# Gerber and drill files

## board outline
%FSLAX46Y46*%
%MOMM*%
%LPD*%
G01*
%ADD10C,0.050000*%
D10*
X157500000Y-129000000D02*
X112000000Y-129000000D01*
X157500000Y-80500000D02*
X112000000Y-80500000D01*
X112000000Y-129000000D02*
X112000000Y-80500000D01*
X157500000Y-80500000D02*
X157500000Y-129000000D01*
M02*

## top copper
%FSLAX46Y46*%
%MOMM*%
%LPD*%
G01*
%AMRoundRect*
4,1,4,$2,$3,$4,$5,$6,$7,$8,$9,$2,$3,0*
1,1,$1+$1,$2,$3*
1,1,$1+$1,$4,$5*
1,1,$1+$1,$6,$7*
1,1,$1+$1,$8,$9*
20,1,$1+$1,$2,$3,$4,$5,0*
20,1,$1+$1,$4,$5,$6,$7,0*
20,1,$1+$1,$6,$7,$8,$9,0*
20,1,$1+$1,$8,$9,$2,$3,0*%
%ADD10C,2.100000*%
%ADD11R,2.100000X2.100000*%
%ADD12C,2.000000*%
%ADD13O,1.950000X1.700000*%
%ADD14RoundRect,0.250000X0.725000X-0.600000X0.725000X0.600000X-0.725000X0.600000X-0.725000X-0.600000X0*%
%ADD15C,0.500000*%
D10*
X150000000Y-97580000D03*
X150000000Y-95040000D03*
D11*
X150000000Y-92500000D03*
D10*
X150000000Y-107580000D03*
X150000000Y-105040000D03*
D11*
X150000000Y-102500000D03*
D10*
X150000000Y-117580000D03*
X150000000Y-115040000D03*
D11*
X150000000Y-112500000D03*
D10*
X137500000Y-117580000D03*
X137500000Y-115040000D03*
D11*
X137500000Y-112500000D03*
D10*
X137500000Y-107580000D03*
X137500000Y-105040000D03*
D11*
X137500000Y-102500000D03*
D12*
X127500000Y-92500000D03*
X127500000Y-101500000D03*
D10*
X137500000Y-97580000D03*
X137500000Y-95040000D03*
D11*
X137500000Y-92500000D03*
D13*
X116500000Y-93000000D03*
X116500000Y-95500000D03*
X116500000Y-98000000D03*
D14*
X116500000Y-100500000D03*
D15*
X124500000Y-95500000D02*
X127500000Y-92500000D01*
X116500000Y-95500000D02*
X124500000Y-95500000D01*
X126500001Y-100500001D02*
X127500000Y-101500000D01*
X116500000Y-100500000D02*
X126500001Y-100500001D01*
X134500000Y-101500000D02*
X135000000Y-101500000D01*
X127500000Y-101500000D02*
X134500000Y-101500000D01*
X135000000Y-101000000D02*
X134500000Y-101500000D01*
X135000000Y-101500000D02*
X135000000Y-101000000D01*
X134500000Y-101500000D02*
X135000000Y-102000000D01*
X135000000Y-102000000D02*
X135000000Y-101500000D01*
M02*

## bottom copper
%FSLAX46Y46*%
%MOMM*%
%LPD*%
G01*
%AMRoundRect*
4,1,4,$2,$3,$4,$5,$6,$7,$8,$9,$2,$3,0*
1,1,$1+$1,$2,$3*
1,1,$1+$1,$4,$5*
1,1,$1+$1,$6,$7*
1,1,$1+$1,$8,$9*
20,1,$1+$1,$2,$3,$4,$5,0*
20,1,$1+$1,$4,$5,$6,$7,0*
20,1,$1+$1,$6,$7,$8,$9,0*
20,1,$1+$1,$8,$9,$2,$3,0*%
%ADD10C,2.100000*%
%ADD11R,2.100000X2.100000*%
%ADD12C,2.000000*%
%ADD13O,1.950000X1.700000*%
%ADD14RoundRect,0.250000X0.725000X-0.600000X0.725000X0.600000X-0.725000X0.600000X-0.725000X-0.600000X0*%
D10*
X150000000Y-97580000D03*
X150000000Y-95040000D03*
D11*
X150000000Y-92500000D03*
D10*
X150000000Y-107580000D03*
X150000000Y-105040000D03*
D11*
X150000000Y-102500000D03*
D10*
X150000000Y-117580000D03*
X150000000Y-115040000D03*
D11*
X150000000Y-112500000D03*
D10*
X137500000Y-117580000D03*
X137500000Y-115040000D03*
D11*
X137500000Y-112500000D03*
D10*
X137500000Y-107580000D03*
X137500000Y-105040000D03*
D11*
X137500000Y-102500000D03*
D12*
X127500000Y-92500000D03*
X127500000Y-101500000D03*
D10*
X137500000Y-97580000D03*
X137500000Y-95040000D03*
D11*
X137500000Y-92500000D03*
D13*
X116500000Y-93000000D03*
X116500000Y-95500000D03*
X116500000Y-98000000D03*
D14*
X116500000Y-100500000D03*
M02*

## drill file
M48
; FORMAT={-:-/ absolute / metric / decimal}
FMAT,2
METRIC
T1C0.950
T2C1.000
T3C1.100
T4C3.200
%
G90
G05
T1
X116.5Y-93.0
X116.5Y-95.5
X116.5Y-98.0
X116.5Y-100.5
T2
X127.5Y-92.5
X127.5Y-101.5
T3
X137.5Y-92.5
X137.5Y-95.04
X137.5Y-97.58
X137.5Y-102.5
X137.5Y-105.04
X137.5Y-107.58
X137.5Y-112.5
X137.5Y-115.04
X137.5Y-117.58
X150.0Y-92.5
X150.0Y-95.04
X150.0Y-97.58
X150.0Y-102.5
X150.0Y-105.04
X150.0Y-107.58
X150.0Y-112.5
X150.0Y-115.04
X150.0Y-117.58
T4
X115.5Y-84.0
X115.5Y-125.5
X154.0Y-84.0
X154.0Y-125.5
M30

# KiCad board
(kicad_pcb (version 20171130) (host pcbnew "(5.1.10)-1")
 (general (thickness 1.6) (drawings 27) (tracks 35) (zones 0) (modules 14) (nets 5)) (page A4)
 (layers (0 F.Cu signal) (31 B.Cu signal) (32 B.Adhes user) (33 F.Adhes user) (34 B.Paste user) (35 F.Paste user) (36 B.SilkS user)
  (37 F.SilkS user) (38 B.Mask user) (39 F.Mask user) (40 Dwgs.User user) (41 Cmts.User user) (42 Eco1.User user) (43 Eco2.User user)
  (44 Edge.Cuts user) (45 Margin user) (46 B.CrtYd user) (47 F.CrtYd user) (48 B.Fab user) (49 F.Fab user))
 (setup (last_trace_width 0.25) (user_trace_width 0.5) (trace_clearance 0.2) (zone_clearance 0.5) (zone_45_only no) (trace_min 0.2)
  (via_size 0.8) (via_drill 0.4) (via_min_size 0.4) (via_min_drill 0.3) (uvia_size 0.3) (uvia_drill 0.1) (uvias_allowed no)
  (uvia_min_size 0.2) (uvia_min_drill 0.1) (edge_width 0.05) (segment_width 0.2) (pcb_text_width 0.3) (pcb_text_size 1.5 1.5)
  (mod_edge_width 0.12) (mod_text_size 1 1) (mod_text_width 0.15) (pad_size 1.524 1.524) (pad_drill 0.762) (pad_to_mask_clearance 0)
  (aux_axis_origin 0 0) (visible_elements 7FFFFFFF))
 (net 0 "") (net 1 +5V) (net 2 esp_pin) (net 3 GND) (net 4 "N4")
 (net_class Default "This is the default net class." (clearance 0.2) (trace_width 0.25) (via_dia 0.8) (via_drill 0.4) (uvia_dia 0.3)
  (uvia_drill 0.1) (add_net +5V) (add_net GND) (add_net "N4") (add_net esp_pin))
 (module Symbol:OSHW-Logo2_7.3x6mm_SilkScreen (layer F.Cu) (at 137.5 124.5)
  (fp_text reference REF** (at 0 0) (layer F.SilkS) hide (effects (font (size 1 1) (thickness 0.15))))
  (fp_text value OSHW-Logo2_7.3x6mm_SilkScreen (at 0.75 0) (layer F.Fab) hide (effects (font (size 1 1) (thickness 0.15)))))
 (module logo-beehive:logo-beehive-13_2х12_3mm (layer F.Cu) (at 123 109.22)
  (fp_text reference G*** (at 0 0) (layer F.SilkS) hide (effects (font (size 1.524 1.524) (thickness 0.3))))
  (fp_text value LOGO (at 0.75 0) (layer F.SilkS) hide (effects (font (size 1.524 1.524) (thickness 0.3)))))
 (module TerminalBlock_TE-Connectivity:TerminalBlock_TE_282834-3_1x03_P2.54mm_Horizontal (layer F.Cu) (at 150 92.5 270)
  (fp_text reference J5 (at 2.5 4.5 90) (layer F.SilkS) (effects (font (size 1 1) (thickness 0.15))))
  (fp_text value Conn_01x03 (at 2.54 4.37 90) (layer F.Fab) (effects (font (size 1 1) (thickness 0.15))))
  (pad 3 thru_hole circle (at 5.08 0 270) (size 2.1 2.1) (drill 1.1) (layers *.Cu *.Mask))
  (pad 2 thru_hole circle (at 2.54 0 270) (size 2.1 2.1) (drill 1.1) (layers *.Cu *.Mask))
  (pad 1 thru_hole rect (at 0 0 270) (size 2.1 2.1) (drill 1.1) (layers *.Cu *.Mask)))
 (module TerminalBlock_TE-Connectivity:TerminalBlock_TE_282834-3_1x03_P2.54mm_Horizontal (layer F.Cu) (at 150 102.5 270)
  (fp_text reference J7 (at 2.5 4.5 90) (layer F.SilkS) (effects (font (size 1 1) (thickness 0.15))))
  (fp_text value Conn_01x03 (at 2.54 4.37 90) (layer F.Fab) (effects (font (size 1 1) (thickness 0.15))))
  (pad 3 thru_hole circle (at 5.08 0 270) (size 2.1 2.1) (drill 1.1) (layers *.Cu *.Mask))
  (pad 2 thru_hole circle (at 2.54 0 270) (size 2.1 2.1) (drill 1.1) (layers *.Cu *.Mask))
  (pad 1 thru_hole rect (at 0 0 270) (size 2.1 2.1) (drill 1.1) (layers *.Cu *.Mask)))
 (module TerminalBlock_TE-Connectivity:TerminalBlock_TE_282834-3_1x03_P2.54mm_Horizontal (layer F.Cu) (at 150 112.5 270)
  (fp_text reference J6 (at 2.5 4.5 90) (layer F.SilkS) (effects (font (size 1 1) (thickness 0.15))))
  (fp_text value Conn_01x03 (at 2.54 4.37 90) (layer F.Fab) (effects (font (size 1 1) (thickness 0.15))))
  (pad 3 thru_hole circle (at 5.08 0 270) (size 2.1 2.1) (drill 1.1) (layers *.Cu *.Mask))
  (pad 2 thru_hole circle (at 2.54 0 270) (size 2.1 2.1) (drill 1.1) (layers *.Cu *.Mask))
  (pad 1 thru_hole rect (at 0 0 270) (size 2.1 2.1) (drill 1.1) (layers *.Cu *.Mask)))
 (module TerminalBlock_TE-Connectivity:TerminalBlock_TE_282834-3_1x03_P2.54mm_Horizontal (layer F.Cu) (at 137.5 112.5 270)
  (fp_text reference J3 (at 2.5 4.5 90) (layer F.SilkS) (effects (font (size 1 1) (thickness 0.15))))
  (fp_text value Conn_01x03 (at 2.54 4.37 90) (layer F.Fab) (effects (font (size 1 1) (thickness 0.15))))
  (pad 3 thru_hole circle (at 5.08 0 270) (size 2.1 2.1) (drill 1.1) (layers *.Cu *.Mask))
  (pad 2 thru_hole circle (at 2.54 0 270) (size 2.1 2.1) (drill 1.1) (layers *.Cu *.Mask))
  (pad 1 thru_hole rect (at 0 0 270) (size 2.1 2.1) (drill 1.1) (layers *.Cu *.Mask)))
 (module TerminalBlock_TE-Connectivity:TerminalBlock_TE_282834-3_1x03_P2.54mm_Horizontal (layer F.Cu) (at 137.5 102.5 270)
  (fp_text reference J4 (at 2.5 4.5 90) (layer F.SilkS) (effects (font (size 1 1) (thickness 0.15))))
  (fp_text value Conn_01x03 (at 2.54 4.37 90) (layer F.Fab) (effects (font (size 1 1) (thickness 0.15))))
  (pad 3 thru_hole circle (at 5.08 0 270) (size 2.1 2.1) (drill 1.1) (layers *.Cu *.Mask))
  (pad 2 thru_hole circle (at 2.54 0 270) (size 2.1 2.1) (drill 1.1) (layers *.Cu *.Mask))
  (pad 1 thru_hole rect (at 0 0 270) (size 2.1 2.1) (drill 1.1) (layers *.Cu *.Mask)))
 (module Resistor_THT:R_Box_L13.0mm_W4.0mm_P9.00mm (layer F.Cu) (at 127.5 101.5 90)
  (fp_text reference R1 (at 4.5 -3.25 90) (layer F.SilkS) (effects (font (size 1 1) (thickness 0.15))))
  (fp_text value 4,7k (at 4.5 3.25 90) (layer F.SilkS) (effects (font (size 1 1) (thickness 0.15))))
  (pad 2 thru_hole circle (at 9 0 90) (size 2 2) (drill 1) (layers *.Cu *.Mask) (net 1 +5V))
  (pad 1 thru_hole circle (at 0 0 90) (size 2 2) (drill 1) (layers *.Cu *.Mask) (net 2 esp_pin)))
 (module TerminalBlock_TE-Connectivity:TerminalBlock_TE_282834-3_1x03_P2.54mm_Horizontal (layer F.Cu) (at 137.5 92.5 270)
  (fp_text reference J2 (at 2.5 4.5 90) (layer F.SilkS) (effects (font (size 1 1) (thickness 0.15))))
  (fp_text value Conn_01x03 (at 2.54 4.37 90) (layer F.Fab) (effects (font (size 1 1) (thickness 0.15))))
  (pad 3 thru_hole circle (at 5.08 0 270) (size 2.1 2.1) (drill 1.1) (layers *.Cu *.Mask))
  (pad 2 thru_hole circle (at 2.54 0 270) (size 2.1 2.1) (drill 1.1) (layers *.Cu *.Mask))
  (pad 1 thru_hole rect (at 0 0 270) (size 2.1 2.1) (drill 1.1) (layers *.Cu *.Mask)))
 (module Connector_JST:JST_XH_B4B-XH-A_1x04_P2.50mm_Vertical (layer F.Cu) (at 116.5 100.5 90)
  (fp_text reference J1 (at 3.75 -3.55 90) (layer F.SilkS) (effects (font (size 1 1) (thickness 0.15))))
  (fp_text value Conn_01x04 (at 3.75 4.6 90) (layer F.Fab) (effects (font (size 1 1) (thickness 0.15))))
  (pad 4 thru_hole oval (at 7.5 0 90) (size 1.7 1.95) (drill 0.95) (layers *.Cu *.Mask))
  (pad 3 thru_hole oval (at 5 0 90) (size 1.7 1.95) (drill 0.95) (layers *.Cu *.Mask) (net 1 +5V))
  (pad 2 thru_hole oval (at 2.5 0 90) (size 1.7 1.95) (drill 0.95) (layers *.Cu *.Mask))
  (pad 1 thru_hole roundrect (at 0 0 90) (size 1.7 1.95) (drill 0.95) (layers *.Cu *.Mask) (roundrect_rratio 0.1470588235294118)
   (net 2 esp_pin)))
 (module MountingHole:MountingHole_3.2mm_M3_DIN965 (layer F.Cu) (at 154 125.5)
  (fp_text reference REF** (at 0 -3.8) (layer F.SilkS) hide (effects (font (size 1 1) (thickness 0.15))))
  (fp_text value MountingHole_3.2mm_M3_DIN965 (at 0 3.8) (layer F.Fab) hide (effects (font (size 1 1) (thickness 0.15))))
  (pad 1 np_thru_hole circle (at 0 0) (size 3.2 3.2) (drill 3.2) (layers *.Cu *.Mask)))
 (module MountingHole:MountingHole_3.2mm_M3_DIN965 (layer F.Cu) (at 154 84)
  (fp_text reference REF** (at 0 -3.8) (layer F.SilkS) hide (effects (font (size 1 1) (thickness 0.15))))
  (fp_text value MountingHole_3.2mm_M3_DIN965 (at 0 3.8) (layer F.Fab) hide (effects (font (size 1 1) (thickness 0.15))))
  (pad 1 np_thru_hole circle (at 0 0) (size 3.2 3.2) (drill 3.2) (layers *.Cu *.Mask)))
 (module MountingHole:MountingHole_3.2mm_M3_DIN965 (layer F.Cu) (at 115.5 125.5)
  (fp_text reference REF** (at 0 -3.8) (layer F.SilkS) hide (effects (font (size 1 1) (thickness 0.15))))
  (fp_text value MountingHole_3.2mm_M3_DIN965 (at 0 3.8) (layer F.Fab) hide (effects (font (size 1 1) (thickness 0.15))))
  (pad 1 np_thru_hole circle (at 0 0) (size 3.2 3.2) (drill 3.2) (layers *.Cu *.Mask)))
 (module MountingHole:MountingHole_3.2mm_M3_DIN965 (layer F.Cu) (at 115.5 84)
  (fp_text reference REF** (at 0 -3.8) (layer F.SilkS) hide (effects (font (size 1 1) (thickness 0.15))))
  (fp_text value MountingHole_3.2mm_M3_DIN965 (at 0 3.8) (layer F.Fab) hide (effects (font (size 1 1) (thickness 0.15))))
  (pad 1 np_thru_hole circle (at 0 0) (size 3.2 3.2) (drill 3.2) (layers *.Cu *.Mask)))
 (gr_line (start 157.5 129) (end 112 129) (layer Edge.Cuts) (width 0.05))
 (gr_line (start 157.5 80.5) (end 112 80.5) (layer Edge.Cuts) (width 0.05))
 (gr_line (start 112 129) (end 112 80.5) (layer Edge.Cuts) (width 0.05))
 (gr_line (start 157.5 80.5) (end 157.5 129) (layer Edge.Cuts) (width 0.05))
 (segment (start 124.5 95.5) (end 127.5 92.5) (width 0.5) (layer F.Cu) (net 1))
 (segment (start 116.5 95.5) (end 124.5 95.5) (width 0.5) (layer F.Cu) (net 1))
 (segment (start 126.500001 100.500001) (end 127.5 101.5) (width 0.5) (layer F.Cu) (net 2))
 (segment (start 116.5 100.5) (end 126.500001 100.500001) (width 0.5) (layer F.Cu) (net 2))
 (segment (start 134.5 101.5) (end 135 101.5) (width 0.5) (layer F.Cu) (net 2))
 (segment (start 127.5 101.5) (end 134.5 101.5) (width 0.5) (layer F.Cu) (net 2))
 (segment (start 135 101) (end 134.5 101.5) (width 0.5) (layer F.Cu) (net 2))
 (segment (start 135 101.5) (end 135 101) (width 0.5) (layer F.Cu) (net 2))
 (segment (start 134.5 101.5) (end 135 102) (width 0.5) (layer F.Cu) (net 2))
 (segment (start 135 102) (end 135 101.5) (width 0.5) (layer F.Cu) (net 2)))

